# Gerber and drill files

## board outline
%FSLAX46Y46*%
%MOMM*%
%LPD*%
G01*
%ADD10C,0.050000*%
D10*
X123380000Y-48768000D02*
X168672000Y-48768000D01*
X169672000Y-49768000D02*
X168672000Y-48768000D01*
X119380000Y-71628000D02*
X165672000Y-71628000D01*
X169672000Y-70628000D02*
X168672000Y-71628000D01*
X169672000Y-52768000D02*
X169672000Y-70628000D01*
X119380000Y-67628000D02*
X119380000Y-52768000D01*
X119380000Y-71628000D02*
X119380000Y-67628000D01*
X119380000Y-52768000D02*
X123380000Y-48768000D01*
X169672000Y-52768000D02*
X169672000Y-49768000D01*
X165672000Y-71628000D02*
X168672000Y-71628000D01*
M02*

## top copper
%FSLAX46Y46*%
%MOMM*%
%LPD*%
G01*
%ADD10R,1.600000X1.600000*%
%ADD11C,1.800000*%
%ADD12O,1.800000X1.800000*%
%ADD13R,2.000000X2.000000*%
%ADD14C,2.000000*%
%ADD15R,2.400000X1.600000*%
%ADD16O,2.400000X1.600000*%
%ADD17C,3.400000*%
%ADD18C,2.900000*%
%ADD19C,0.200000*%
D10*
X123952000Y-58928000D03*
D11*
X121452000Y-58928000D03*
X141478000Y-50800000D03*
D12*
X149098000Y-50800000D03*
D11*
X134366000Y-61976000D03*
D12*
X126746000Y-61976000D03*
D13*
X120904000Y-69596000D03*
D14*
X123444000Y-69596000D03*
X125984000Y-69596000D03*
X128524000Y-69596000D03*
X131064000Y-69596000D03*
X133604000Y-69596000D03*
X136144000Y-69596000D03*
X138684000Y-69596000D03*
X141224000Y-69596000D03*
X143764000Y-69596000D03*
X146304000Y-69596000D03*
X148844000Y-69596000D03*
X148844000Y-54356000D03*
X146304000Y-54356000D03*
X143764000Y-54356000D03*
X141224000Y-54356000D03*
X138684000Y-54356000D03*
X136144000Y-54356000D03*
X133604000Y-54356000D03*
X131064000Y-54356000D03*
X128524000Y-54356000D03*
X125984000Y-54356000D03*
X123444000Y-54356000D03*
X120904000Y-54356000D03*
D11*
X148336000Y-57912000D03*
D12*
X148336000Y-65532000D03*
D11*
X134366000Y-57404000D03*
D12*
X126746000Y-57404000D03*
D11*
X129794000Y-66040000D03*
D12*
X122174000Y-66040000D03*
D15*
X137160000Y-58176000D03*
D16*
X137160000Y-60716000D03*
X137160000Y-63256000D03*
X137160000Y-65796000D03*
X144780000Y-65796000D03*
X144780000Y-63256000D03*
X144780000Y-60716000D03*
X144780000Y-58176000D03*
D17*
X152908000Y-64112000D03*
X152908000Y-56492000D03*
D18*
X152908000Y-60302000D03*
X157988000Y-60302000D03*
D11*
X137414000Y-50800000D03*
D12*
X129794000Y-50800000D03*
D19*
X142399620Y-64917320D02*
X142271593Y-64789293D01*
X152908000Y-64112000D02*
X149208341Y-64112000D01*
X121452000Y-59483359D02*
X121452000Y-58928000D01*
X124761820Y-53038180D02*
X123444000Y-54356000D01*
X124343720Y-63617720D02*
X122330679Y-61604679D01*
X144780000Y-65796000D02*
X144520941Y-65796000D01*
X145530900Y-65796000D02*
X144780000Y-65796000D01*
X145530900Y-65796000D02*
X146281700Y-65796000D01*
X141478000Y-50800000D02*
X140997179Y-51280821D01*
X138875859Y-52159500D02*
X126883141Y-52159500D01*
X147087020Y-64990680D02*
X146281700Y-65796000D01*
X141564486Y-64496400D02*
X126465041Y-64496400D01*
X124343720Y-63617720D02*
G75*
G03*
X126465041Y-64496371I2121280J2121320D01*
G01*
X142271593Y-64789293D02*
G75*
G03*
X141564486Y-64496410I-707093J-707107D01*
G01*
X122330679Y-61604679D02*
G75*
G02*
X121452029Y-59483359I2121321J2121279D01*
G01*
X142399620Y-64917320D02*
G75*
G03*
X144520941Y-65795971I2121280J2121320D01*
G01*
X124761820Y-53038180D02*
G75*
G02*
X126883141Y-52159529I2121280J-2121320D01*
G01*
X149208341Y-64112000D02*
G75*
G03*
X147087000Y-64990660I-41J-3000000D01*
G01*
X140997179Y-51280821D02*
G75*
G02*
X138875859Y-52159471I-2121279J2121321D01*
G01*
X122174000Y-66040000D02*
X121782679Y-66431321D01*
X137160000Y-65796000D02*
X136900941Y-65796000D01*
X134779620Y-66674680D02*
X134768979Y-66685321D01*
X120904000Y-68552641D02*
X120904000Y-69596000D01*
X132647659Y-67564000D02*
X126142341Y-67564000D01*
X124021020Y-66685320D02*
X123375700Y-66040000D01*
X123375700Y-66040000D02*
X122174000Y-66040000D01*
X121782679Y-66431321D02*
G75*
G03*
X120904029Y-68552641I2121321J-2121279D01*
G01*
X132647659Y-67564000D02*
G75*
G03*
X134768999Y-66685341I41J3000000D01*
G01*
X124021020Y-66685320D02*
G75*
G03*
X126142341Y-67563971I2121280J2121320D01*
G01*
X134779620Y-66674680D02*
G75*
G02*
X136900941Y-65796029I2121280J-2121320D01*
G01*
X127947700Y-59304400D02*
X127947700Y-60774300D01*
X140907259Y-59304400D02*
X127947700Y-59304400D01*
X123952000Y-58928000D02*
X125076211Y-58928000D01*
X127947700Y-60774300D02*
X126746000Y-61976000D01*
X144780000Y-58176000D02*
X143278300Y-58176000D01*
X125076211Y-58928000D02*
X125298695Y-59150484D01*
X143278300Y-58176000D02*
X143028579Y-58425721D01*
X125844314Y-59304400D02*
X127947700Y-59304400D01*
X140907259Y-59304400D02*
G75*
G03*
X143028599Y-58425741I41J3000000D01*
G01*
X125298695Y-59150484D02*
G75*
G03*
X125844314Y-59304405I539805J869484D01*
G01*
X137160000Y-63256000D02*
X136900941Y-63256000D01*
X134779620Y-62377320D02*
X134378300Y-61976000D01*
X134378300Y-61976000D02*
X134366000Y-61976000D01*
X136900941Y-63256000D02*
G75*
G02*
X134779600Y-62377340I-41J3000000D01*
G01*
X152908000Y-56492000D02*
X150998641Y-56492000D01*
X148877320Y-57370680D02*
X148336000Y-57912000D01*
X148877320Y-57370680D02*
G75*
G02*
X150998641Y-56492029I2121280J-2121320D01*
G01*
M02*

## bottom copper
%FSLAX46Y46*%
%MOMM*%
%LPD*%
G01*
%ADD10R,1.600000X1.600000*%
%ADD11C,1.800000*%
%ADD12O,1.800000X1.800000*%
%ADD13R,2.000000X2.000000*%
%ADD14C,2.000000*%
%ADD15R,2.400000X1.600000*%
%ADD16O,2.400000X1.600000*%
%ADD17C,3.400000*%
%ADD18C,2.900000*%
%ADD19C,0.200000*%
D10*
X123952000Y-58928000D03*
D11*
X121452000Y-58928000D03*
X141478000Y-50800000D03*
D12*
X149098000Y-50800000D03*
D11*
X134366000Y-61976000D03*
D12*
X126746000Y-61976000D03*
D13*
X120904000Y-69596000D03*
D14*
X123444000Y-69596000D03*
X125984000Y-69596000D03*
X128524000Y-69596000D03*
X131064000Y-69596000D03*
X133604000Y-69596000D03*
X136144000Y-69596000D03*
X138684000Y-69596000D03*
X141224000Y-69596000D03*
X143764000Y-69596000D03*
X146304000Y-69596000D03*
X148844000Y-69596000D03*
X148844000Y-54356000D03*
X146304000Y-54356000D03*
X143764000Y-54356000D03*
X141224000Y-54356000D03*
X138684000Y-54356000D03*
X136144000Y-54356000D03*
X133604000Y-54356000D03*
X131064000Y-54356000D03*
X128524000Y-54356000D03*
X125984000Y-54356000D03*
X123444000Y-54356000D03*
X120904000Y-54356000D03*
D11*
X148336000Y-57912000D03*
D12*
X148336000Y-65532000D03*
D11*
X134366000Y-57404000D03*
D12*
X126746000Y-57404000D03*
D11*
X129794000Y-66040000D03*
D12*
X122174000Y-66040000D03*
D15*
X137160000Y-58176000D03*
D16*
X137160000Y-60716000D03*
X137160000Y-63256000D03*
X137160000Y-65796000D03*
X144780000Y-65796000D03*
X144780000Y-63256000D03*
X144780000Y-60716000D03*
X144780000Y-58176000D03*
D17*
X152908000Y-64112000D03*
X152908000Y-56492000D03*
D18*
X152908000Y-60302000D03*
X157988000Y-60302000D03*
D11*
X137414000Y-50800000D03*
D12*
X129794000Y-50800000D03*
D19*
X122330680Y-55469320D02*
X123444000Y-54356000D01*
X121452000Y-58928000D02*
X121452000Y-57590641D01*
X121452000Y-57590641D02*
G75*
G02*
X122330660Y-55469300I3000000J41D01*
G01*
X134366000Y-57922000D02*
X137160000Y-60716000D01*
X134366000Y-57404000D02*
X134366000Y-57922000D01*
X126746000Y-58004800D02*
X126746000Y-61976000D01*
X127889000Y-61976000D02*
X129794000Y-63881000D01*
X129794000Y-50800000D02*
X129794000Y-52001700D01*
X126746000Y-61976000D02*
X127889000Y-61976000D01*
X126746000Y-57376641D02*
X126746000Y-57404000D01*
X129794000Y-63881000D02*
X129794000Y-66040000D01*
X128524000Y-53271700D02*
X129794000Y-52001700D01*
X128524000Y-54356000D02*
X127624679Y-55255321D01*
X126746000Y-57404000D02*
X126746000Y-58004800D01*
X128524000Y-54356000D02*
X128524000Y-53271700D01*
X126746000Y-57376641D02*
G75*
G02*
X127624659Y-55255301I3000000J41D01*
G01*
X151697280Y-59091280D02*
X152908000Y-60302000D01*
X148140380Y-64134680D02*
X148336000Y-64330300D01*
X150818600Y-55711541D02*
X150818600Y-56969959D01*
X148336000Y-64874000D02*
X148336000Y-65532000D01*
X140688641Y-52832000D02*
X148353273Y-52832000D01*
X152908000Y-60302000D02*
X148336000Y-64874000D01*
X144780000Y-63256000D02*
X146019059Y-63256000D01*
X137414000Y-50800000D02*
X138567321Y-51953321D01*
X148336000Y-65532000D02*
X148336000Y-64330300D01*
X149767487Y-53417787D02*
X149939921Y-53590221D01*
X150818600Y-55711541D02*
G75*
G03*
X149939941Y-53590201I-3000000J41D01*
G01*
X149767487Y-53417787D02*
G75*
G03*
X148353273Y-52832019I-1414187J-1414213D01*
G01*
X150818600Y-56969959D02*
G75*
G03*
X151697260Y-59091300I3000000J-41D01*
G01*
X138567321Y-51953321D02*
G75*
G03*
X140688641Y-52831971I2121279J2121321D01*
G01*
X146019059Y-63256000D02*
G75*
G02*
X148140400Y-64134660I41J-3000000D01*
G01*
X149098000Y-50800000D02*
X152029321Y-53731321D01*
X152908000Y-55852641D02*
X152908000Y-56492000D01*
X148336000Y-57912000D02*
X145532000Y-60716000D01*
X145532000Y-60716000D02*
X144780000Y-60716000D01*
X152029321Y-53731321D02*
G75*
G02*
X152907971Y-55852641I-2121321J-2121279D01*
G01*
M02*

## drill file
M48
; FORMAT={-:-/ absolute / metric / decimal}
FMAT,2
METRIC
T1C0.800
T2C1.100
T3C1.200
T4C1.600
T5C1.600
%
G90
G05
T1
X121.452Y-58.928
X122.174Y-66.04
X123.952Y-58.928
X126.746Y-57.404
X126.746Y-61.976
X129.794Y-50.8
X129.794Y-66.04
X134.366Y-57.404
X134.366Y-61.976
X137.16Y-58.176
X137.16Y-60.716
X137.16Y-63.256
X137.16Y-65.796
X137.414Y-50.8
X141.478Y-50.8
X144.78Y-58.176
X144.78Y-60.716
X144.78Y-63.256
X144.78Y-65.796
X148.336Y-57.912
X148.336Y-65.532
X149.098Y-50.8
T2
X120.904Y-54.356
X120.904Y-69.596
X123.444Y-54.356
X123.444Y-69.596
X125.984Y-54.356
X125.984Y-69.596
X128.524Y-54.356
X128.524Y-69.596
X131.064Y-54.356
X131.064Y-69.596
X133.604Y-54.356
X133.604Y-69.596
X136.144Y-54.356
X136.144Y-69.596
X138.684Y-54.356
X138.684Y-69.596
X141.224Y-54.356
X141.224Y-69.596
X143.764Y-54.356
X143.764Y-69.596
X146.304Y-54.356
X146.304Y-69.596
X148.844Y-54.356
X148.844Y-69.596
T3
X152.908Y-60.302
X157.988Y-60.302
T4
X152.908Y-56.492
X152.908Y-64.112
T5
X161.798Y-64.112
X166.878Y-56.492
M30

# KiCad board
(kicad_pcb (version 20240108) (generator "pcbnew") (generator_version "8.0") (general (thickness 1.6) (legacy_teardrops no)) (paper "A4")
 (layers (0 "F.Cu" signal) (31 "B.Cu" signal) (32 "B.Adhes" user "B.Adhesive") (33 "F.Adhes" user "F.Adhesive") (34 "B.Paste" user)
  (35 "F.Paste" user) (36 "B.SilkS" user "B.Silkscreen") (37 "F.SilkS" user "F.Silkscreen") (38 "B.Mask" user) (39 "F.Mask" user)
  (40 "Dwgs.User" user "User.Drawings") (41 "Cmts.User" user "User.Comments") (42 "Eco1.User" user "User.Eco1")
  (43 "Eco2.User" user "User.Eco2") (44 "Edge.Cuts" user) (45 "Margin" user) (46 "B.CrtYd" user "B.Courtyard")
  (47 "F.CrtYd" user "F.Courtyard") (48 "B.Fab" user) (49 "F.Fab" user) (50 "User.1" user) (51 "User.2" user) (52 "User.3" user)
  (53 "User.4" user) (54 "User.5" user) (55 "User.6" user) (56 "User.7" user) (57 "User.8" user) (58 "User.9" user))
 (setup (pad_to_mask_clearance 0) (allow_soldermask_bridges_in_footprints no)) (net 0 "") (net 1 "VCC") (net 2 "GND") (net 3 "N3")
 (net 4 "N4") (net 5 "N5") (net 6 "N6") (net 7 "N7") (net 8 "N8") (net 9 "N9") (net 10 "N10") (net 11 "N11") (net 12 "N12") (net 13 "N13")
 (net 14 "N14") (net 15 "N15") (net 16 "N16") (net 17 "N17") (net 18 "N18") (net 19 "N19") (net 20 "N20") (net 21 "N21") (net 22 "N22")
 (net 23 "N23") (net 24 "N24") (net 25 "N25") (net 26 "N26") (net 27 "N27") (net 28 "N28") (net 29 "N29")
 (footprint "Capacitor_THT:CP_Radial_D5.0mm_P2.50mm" (layer "F.Cu") (at 123.952 58.928 180)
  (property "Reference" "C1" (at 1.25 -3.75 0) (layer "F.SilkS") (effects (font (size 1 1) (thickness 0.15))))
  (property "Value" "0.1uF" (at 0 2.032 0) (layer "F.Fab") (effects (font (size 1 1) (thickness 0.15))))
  (pad "1" thru_hole rect (at 0 0 180) (size 1.6 1.6) (drill 0.8) (layers "*.Cu" "*.Mask") (remove_unused_layers no) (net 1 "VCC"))
  (pad "2" thru_hole circle (at 2.5 0 180) (size 1.8 1.8) (drill 0.8) (layers "*.Cu" "*.Mask") (remove_unused_layers no) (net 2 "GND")))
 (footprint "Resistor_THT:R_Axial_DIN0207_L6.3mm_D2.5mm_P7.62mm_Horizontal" (layer "F.Cu") (at 141.478 50.8)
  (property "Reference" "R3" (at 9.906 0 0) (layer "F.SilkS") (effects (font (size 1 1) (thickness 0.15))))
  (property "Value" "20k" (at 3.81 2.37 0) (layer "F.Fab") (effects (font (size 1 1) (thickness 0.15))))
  (pad "1" thru_hole circle (at 0 0) (size 1.8 1.8) (drill 0.8) (layers "*.Cu" "*.Mask") (remove_unused_layers no) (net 2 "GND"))
  (pad "2" thru_hole oval (at 7.62 0) (size 1.8 1.8) (drill 0.8) (layers "*.Cu" "*.Mask") (remove_unused_layers no) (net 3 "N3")))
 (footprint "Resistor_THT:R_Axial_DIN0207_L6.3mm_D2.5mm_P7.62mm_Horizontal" (layer "F.Cu") (at 134.366 61.976 180)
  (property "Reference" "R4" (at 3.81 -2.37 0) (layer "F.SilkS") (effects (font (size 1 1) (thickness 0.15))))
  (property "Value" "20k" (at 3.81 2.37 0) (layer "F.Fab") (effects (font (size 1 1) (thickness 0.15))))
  (pad "1" thru_hole circle (at 0 0 180) (size 1.8 1.8) (drill 0.8) (layers "*.Cu" "*.Mask") (remove_unused_layers no) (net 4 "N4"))
  (pad "2" thru_hole oval (at 7.62 0 180) (size 1.8 1.8) (drill 0.8) (layers "*.Cu" "*.Mask") (remove_unused_layers no) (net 1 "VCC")))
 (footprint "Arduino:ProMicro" (layer "F.Cu") (at 134.874 61.976)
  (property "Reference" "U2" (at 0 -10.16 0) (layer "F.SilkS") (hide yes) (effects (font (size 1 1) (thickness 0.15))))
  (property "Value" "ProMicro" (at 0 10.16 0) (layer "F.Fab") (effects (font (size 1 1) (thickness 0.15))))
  (pad "1" thru_hole rect (at -13.97 7.62) (size 2 2) (drill 1.1) (layers "*.Cu" "*.Mask" "F.SilkS") (remove_unused_layers no) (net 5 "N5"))
  (pad "2" thru_hole circle (at -11.43 7.62) (size 2 2) (drill 1.1) (layers "*.Cu" "*.Mask" "F.SilkS") (remove_unused_layers no)
   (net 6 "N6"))
  (pad "3" thru_hole circle (at -8.89 7.62) (size 2 2) (drill 1.1) (layers "*.Cu" "*.Mask" "F.SilkS") (remove_unused_layers no) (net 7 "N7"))
  (pad "4" thru_hole circle (at -6.35 7.62) (size 2 2) (drill 1.1) (layers "*.Cu" "*.Mask" "F.SilkS") (remove_unused_layers no) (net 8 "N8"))
  (pad "5" thru_hole circle (at -3.81 7.62) (size 2 2) (drill 1.1) (layers "*.Cu" "*.Mask" "F.SilkS") (remove_unused_layers no) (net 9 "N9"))
  (pad "6" thru_hole circle (at -1.27 7.62) (size 2 2) (drill 1.1) (layers "*.Cu" "*.Mask" "F.SilkS") (remove_unused_layers no)
   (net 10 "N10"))
  (pad "7" thru_hole circle (at 1.27 7.62) (size 2 2) (drill 1.1) (layers "*.Cu" "*.Mask" "F.SilkS") (remove_unused_layers no)
   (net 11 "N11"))
  (pad "8" thru_hole circle (at 3.81 7.62) (size 2 2) (drill 1.1) (layers "*.Cu" "*.Mask" "F.SilkS") (remove_unused_layers no)
   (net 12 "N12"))
  (pad "9" thru_hole circle (at 6.35 7.62) (size 2 2) (drill 1.1) (layers "*.Cu" "*.Mask" "F.SilkS") (remove_unused_layers no)
   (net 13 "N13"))
  (pad "10" thru_hole circle (at 8.89 7.62) (size 2 2) (drill 1.1) (layers "*.Cu" "*.Mask" "F.SilkS") (remove_unused_layers no)
   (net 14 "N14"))
  (pad "11" thru_hole circle (at 11.43 7.62) (size 2 2) (drill 1.1) (layers "*.Cu" "*.Mask" "F.SilkS") (remove_unused_layers no)
   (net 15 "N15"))
  (pad "12" thru_hole circle (at 13.97 7.62) (size 2 2) (drill 1.1) (layers "*.Cu" "*.Mask" "F.SilkS") (remove_unused_layers no)
   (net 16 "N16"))
  (pad "13" thru_hole circle (at 13.97 -7.62) (size 2 2) (drill 1.1) (layers "*.Cu" "*.Mask" "F.SilkS") (remove_unused_layers no)
   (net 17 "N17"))
  (pad "14" thru_hole circle (at 11.43 -7.62) (size 2 2) (drill 1.1) (layers "*.Cu" "*.Mask" "F.SilkS") (remove_unused_layers no)
   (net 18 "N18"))
  (pad "15" thru_hole circle (at 8.89 -7.62) (size 2 2) (drill 1.1) (layers "*.Cu" "*.Mask" "F.SilkS") (remove_unused_layers no)
   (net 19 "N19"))
  (pad "16" thru_hole circle (at 6.35 -7.62) (size 2 2) (drill 1.1) (layers "*.Cu" "*.Mask" "F.SilkS") (remove_unused_layers no)
   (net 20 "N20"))
  (pad "17" thru_hole circle (at 3.81 -7.62) (size 2 2) (drill 1.1) (layers "*.Cu" "*.Mask" "F.SilkS") (remove_unused_layers no)
   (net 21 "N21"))
  (pad "18" thru_hole circle (at 1.27 -7.62) (size 2 2) (drill 1.1) (layers "*.Cu" "*.Mask" "F.SilkS") (remove_unused_layers no)
   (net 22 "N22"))
  (pad "19" thru_hole circle (at -1.27 -7.62) (size 2 2) (drill 1.1) (layers "*.Cu" "*.Mask" "F.SilkS") (remove_unused_layers no)
   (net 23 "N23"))
  (pad "20" thru_hole circle (at -3.81 -7.62) (size 2 2) (drill 1.1) (layers "*.Cu" "*.Mask" "F.SilkS") (remove_unused_layers no)
   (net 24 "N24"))
  (pad "21" thru_hole circle (at -6.35 -7.62) (size 2 2) (drill 1.1) (layers "*.Cu" "*.Mask" "F.SilkS") (remove_unused_layers no)
   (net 1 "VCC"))
  (pad "22" thru_hole circle (at -8.89 -7.62) (size 2 2) (drill 1.1) (layers "*.Cu" "*.Mask" "F.SilkS") (remove_unused_layers no)
   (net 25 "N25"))
  (pad "23" thru_hole circle (at -11.43 -7.62) (size 2 2) (drill 1.1) (layers "*.Cu" "*.Mask" "F.SilkS") (remove_unused_layers no)
   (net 2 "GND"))
  (pad "24" thru_hole circle (at -13.97 -7.62) (size 2 2) (drill 1.1) (layers "*.Cu" "*.Mask" "F.SilkS") (remove_unused_layers no)
   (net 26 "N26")))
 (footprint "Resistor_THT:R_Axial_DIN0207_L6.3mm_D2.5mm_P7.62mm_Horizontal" (layer "F.Cu") (at 148.336 57.912 -90)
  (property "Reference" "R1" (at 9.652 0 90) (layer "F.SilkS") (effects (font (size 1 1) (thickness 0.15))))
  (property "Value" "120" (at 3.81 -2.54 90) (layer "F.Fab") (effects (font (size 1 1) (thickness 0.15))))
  (pad "1" thru_hole circle (at 0 0 270) (size 1.8 1.8) (drill 0.8) (layers "*.Cu" "*.Mask") (remove_unused_layers no) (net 3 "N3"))
  (pad "2" thru_hole oval (at 7.62 0 270) (size 1.8 1.8) (drill 0.8) (layers "*.Cu" "*.Mask") (remove_unused_layers no) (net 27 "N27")))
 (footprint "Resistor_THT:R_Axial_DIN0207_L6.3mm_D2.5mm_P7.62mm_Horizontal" (layer "F.Cu") (at 134.366 57.404 180)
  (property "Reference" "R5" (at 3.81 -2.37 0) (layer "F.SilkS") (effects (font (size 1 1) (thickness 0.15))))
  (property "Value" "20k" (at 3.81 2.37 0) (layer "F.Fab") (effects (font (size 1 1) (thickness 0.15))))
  (pad "1" thru_hole circle (at 0 0 180) (size 1.8 1.8) (drill 0.8) (layers "*.Cu" "*.Mask") (remove_unused_layers no) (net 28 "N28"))
  (pad "2" thru_hole oval (at 7.62 0 180) (size 1.8 1.8) (drill 0.8) (layers "*.Cu" "*.Mask") (remove_unused_layers no) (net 1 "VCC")))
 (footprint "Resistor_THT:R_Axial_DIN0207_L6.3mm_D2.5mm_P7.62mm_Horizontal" (layer "F.Cu") (at 129.794 66.04 180)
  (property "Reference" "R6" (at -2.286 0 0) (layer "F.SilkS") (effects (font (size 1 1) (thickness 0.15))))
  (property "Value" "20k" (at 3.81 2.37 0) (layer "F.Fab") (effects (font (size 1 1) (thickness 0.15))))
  (pad "1" thru_hole circle (at 0 0 180) (size 1.8 1.8) (drill 0.8) (layers "*.Cu" "*.Mask") (remove_unused_layers no) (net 1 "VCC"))
  (pad "2" thru_hole oval (at 7.62 0 180) (size 1.8 1.8) (drill 0.8) (layers "*.Cu" "*.Mask") (remove_unused_layers no) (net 5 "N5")))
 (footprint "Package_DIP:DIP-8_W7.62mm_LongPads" (layer "F.Cu") (at 137.16 58.176)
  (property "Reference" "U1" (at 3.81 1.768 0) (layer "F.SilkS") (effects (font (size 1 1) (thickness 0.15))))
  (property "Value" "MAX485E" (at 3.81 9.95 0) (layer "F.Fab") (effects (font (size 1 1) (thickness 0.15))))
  (pad "1" thru_hole rect (at 0 0) (size 2.4 1.6) (drill 0.8) (layers "*.Cu" "*.Mask") (remove_unused_layers no) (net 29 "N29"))
  (pad "2" thru_hole oval (at 0 2.54) (size 2.4 1.6) (drill 0.8) (layers "*.Cu" "*.Mask") (remove_unused_layers no) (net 28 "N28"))
  (pad "3" thru_hole oval (at 0 5.08) (size 2.4 1.6) (drill 0.8) (layers "*.Cu" "*.Mask") (remove_unused_layers no) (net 4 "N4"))
  (pad "4" thru_hole oval (at 0 7.62) (size 2.4 1.6) (drill 0.8) (layers "*.Cu" "*.Mask") (remove_unused_layers no) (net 5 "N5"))
  (pad "5" thru_hole oval (at 7.62 7.62) (size 2.4 1.6) (drill 0.8) (layers "*.Cu" "*.Mask") (remove_unused_layers no) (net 2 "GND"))
  (pad "6" thru_hole oval (at 7.62 5.08) (size 2.4 1.6) (drill 0.8) (layers "*.Cu" "*.Mask") (remove_unused_layers no) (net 27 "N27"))
  (pad "7" thru_hole oval (at 7.62 2.54) (size 2.4 1.6) (drill 0.8) (layers "*.Cu" "*.Mask") (remove_unused_layers no) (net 3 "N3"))
  (pad "8" thru_hole oval (at 7.62 0) (size 2.4 1.6) (drill 0.8) (layers "*.Cu" "*.Mask") (remove_unused_layers no) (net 1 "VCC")))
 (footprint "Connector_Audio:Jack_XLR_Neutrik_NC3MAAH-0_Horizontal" (layer "F.Cu") (at 152.908 64.112 90)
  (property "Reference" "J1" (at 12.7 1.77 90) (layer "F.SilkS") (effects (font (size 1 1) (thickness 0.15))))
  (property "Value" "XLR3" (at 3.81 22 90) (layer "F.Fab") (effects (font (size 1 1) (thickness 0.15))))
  (pad "" np_thru_hole circle (at 0 8.89 90) (size 1.6 1.6) (drill 1.6) (layers "*.Cu" "*.Mask"))
  (pad "" np_thru_hole circle (at 7.62 13.97 90) (size 1.6 1.6) (drill 1.6) (layers "*.Cu" "*.Mask"))
  (pad "1" thru_hole circle (at 0 0 90) (size 3.4 3.4) (drill 1.6) (layers "*.Cu" "*.Mask") (remove_unused_layers no) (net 2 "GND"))
  (pad "2" thru_hole circle (at 7.62 0 90) (size 3.4 3.4) (drill 1.6) (layers "*.Cu" "*.Mask") (remove_unused_layers no) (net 3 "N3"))
  (pad "3" thru_hole circle (at 3.81 0 90) (size 2.9 2.9) (drill 1.2) (layers "*.Cu" "*.Mask") (remove_unused_layers no) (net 27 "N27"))
  (pad "G" thru_hole circle (at 3.81 5.08 90) (size 2.9 2.9) (drill 1.2) (layers "*.Cu" "*.Mask") (remove_unused_layers no)))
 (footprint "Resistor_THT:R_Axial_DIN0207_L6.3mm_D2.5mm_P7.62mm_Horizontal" (layer "F.Cu") (at 137.414 50.8 180)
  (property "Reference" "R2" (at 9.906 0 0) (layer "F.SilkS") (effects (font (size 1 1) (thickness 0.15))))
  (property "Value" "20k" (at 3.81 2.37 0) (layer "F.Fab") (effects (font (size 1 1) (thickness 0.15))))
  (pad "1" thru_hole circle (at 0 0 180) (size 1.8 1.8) (drill 0.8) (layers "*.Cu" "*.Mask") (remove_unused_layers no) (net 27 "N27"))
  (pad "2" thru_hole oval (at 7.62 0 180) (size 1.8 1.8) (drill 0.8) (layers "*.Cu" "*.Mask") (remove_unused_layers no) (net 1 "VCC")))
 (gr_line (start 123.38 48.768) (end 168.672 48.768) (stroke (width 0.05) (type default)) (layer "Edge.Cuts"))
 (gr_line (start 169.672 49.768) (end 168.672 48.768) (stroke (width 0.05) (type default)) (layer "Edge.Cuts"))
 (gr_line (start 119.38 71.628) (end 165.672 71.628) (stroke (width 0.05) (type default)) (layer "Edge.Cuts"))
 (gr_line (start 169.672 70.628) (end 168.672 71.628) (stroke (width 0.05) (type default)) (layer "Edge.Cuts"))
 (gr_line (start 169.672 52.768) (end 169.672 70.628) (stroke (width 0.05) (type default)) (layer "Edge.Cuts"))
 (gr_line (start 119.38 67.628) (end 119.38 52.768) (stroke (width 0.05) (type default)) (layer "Edge.Cuts"))
 (gr_line (start 119.38 71.628) (end 119.38 67.628) (stroke (width 0.05) (type default)) (layer "Edge.Cuts"))
 (gr_line (start 119.38 52.768) (end 123.38 48.768) (stroke (width 0.05) (type default)) (layer "Edge.Cuts"))
 (gr_line (start 169.672 52.768) (end 169.672 49.768) (stroke (width 0.05) (type default)) (layer "Edge.Cuts"))
 (gr_line (start 165.672 71.628) (end 168.672 71.628) (stroke (width 0.05) (type default)) (layer "Edge.Cuts"))
 (segment (start 142.39962 64.91732) (end 142.271593 64.789293) (width 0.2) (layer "F.Cu") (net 2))
 (segment (start 152.908 64.112) (end 149.208341 64.112) (width 0.2) (layer "F.Cu") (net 2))
 (segment (start 121.452 59.483359) (end 121.452 58.928) (width 0.2) (layer "F.Cu") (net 2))
 (segment (start 124.76182 53.03818) (end 123.444 54.356) (width 0.2) (layer "F.Cu") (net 2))
 (segment (start 124.34372 63.61772) (end 122.330679 61.604679) (width 0.2) (layer "F.Cu") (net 2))
 (segment (start 144.78 65.796) (end 144.520941 65.796) (width 0.2) (layer "F.Cu") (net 2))
 (segment (start 145.5309 65.796) (end 144.78 65.796) (width 0.2) (layer "F.Cu") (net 2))
 (segment (start 145.5309 65.796) (end 146.2817 65.796) (width 0.2) (layer "F.Cu") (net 2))
 (segment (start 141.478 50.8) (end 140.997179 51.280821) (width 0.2) (layer "F.Cu") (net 2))
 (segment (start 138.875859 52.1595) (end 126.883141 52.1595) (width 0.2) (layer "F.Cu") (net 2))
 (segment (start 147.08702 64.99068) (end 146.2817 65.796) (width 0.2) (layer "F.Cu") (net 2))
 (segment (start 141.564486 64.4964) (end 126.465041 64.4964) (width 0.2) (layer "F.Cu") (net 2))
 (arc (start 124.34372 63.61772) (mid 125.31699 64.268039) (end 126.465041 64.4964) (width 0.2) (layer "F.Cu") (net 2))
 (arc (start 142.271593 64.789293) (mid 141.94717 64.57252) (end 141.564486 64.4964) (width 0.2) (layer "F.Cu") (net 2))
 (arc (start 122.330679 61.604679) (mid 121.680361 60.631409) (end 121.452 59.483359) (width 0.2) (layer "F.Cu") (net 2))
 (arc (start 142.39962 64.91732) (mid 143.37289 65.567639) (end 144.520941 65.796) (width 0.2) (layer "F.Cu") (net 2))
 (arc (start 124.76182 53.03818) (mid 125.73509 52.387861) (end 126.883141 52.1595) (width 0.2) (layer "F.Cu") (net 2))
 (arc (start 149.208341 64.112) (mid 148.06029 64.340362) (end 147.08702 64.99068) (width 0.2) (layer "F.Cu") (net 2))
 (arc (start 140.997179 51.280821) (mid 140.023909 51.931139) (end 138.875859 52.1595) (width 0.2) (layer "F.Cu") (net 2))
 (segment (start 122.33068 55.46932) (end 123.444 54.356) (width 0.2) (layer "B.Cu") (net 2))
 (segment (start 121.452 58.928) (end 121.452 57.590641) (width 0.2) (layer "B.Cu") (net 2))
 (arc (start 121.452 57.590641) (mid 121.680362 56.44259) (end 122.33068 55.46932) (width 0.2) (layer "B.Cu") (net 2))
 (segment (start 134.366 57.922) (end 137.16 60.716) (width 0.2) (layer "B.Cu") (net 28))
 (segment (start 134.366 57.404) (end 134.366 57.922) (width 0.2) (layer "B.Cu") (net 28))
 (segment (start 122.174 66.04) (end 121.782679 66.431321) (width 0.2) (layer "F.Cu") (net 5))
 (segment (start 137.16 65.796) (end 136.900941 65.796) (width 0.2) (layer "F.Cu") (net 5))
 (segment (start 134.77962 66.67468) (end 134.768979 66.685321) (width 0.2) (layer "F.Cu") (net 5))
 (segment (start 120.904 68.552641) (end 120.904 69.596) (width 0.2) (layer "F.Cu") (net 5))
 (segment (start 132.647659 67.564) (end 126.142341 67.564) (width 0.2) (layer "F.Cu") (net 5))
 (segment (start 124.02102 66.68532) (end 123.3757 66.04) (width 0.2) (layer "F.Cu") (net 5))
 (segment (start 123.3757 66.04) (end 122.174 66.04) (width 0.2) (layer "F.Cu") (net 5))
 (arc (start 121.782679 66.431321) (mid 121.132361 67.404591) (end 120.904 68.552641) (width 0.2) (layer "F.Cu") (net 5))
 (arc (start 132.647659 67.564) (mid 133.795709 67.335639) (end 134.768979 66.685321) (width 0.2) (layer "F.Cu") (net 5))
 (arc (start 124.02102 66.68532) (mid 124.99429 67.335639) (end 126.142341 67.564) (width 0.2) (layer "F.Cu") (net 5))
 (arc (start 134.77962 66.67468) (mid 135.75289 66.024361) (end 136.900941 65.796) (width 0.2) (layer "F.Cu") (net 5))
 (segment (start 127.9477 59.3044) (end 127.9477 60.7743) (width 0.2) (layer "F.Cu") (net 1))
 (segment (start 140.907259 59.3044) (end 127.9477 59.3044) (width 0.2) (layer "F.Cu") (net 1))
 (segment (start 123.952 58.928) (end 125.076211 58.928) (width 0.2) (layer "F.Cu") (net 1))
 (segment (start 127.9477 60.7743) (end 126.746 61.976) (width 0.2) (layer "F.Cu") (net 1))
 (segment (start 144.78 58.176) (end 143.2783 58.176) (width 0.2) (layer "F.Cu") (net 1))
 (segment (start 125.076211 58.928) (end 125.298695 59.150484) (width 0.2) (layer "F.Cu") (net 1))
 (segment (start 143.2783 58.176) (end 143.028579 58.425721) (width 0.2) (layer "F.Cu") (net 1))
 (segment (start 125.844314 59.3044) (end 127.9477 59.3044) (width 0.2) (layer "F.Cu") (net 1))
 (arc (start 140.907259 59.3044) (mid 142.055309 59.076039) (end 143.028579 58.425721) (width 0.2) (layer "F.Cu") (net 1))
 (arc (start 125.298695 59.150484) (mid 125.560902 59.26605) (end 125.844314 59.3044) (width 0.2) (layer "F.Cu") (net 1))
 (segment (start 126.746 58.0048) (end 126.746 61.976) (width 0.2) (layer "B.Cu") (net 1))
 (segment (start 127.889 61.976) (end 129.794 63.881) (width 0.2) (layer "B.Cu") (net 1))
 (segment (start 129.794 50.8) (end 129.794 52.0017) (width 0.2) (layer "B.Cu") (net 1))
 (segment (start 126.746 61.976) (end 127.889 61.976) (width 0.2) (layer "B.Cu") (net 1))
 (segment (start 126.746 57.376641) (end 126.746 57.404) (width 0.2) (layer "B.Cu") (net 1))
 (segment (start 129.794 63.881) (end 129.794 66.04) (width 0.2) (layer "B.Cu") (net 1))
 (segment (start 128.524 53.2717) (end 129.794 52.0017) (width 0.2) (layer "B.Cu") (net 1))
 (segment (start 128.524 54.356) (end 127.624679 55.255321) (width 0.2) (layer "B.Cu") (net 1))
 (segment (start 126.746 57.404) (end 126.746 58.0048) (width 0.2) (layer "B.Cu") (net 1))
 (segment (start 128.524 54.356) (end 128.524 53.2717) (width 0.2) (layer "B.Cu") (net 1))
 (arc (start 126.746 57.376641) (mid 126.974361 56.228591) (end 127.624679 55.255321) (width 0.2) (layer "B.Cu") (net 1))
 (segment (start 151.69728 59.09128) (end 152.908 60.302) (width 0.2) (layer "B.Cu") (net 27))
 (segment (start 148.14038 64.13468) (end 148.336 64.3303) (width 0.2) (layer "B.Cu") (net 27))
 (segment (start 150.8186 55.711541) (end 150.8186 56.969959) (width 0.2) (layer "B.Cu") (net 27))
 (segment (start 148.336 64.874) (end 148.336 65.532) (width 0.2) (layer "B.Cu") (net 27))
 (segment (start 140.688641 52.832) (end 148.353273 52.832) (width 0.2) (layer "B.Cu") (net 27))
 (segment (start 152.908 60.302) (end 148.336 64.874) (width 0.2) (layer "B.Cu") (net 27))
 (segment (start 144.78 63.256) (end 146.019059 63.256) (width 0.2) (layer "B.Cu") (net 27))
 (segment (start 137.414 50.8) (end 138.567321 51.953321) (width 0.2) (layer "B.Cu") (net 27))
 (segment (start 148.336 65.532) (end 148.336 64.3303) (width 0.2) (layer "B.Cu") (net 27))
 (segment (start 149.767487 53.417787) (end 149.939921 53.590221) (width 0.2) (layer "B.Cu") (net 27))
 (arc (start 150.8186 55.711541) (mid 150.590239 54.563491) (end 149.939921 53.590221) (width 0.2) (layer "B.Cu") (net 27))
 (arc (start 149.767487 53.417787) (mid 149.11864 52.984241) (end 148.353273 52.832) (width 0.2) (layer "B.Cu") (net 27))
 (arc (start 150.8186 56.969959) (mid 151.046962 58.11801) (end 151.69728 59.09128) (width 0.2) (layer "B.Cu") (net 27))
 (arc (start 138.567321 51.953321) (mid 139.540591 52.603639) (end 140.688641 52.832) (width 0.2) (layer "B.Cu") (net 27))
 (arc (start 146.019059 63.256) (mid 147.16711 63.484362) (end 148.14038 64.13468) (width 0.2) (layer "B.Cu") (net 27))
 (segment (start 137.16 63.256) (end 136.900941 63.256) (width 0.2) (layer "F.Cu") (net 4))
 (segment (start 134.77962 62.37732) (end 134.3783 61.976) (width 0.2) (layer "F.Cu") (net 4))
 (segment (start 134.3783 61.976) (end 134.366 61.976) (width 0.2) (layer "F.Cu") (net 4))
 (arc (start 136.900941 63.256) (mid 135.75289 63.027638) (end 134.77962 62.37732) (width 0.2) (layer "F.Cu") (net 4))
 (segment (start 152.908 56.492) (end 150.998641 56.492) (width 0.2) (layer "F.Cu") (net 3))
 (segment (start 148.87732 57.37068) (end 148.336 57.912) (width 0.2) (layer "F.Cu") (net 3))
 (arc (start 148.87732 57.37068) (mid 149.85059 56.720361) (end 150.998641 56.492) (width 0.2) (layer "F.Cu") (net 3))
 (segment (start 149.098 50.8) (end 152.029321 53.731321) (width 0.2) (layer "B.Cu") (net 3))
 (segment (start 152.908 55.852641) (end 152.908 56.492) (width 0.2) (layer "B.Cu") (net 3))
 (segment (start 148.336 57.912) (end 145.532 60.716) (width 0.2) (layer "B.Cu") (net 3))
 (segment (start 145.532 60.716) (end 144.78 60.716) (width 0.2) (layer "B.Cu") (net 3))
 (arc (start 152.029321 53.731321) (mid 152.679639 54.704591) (end 152.908 55.852641) (width 0.2) (layer "B.Cu") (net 3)))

